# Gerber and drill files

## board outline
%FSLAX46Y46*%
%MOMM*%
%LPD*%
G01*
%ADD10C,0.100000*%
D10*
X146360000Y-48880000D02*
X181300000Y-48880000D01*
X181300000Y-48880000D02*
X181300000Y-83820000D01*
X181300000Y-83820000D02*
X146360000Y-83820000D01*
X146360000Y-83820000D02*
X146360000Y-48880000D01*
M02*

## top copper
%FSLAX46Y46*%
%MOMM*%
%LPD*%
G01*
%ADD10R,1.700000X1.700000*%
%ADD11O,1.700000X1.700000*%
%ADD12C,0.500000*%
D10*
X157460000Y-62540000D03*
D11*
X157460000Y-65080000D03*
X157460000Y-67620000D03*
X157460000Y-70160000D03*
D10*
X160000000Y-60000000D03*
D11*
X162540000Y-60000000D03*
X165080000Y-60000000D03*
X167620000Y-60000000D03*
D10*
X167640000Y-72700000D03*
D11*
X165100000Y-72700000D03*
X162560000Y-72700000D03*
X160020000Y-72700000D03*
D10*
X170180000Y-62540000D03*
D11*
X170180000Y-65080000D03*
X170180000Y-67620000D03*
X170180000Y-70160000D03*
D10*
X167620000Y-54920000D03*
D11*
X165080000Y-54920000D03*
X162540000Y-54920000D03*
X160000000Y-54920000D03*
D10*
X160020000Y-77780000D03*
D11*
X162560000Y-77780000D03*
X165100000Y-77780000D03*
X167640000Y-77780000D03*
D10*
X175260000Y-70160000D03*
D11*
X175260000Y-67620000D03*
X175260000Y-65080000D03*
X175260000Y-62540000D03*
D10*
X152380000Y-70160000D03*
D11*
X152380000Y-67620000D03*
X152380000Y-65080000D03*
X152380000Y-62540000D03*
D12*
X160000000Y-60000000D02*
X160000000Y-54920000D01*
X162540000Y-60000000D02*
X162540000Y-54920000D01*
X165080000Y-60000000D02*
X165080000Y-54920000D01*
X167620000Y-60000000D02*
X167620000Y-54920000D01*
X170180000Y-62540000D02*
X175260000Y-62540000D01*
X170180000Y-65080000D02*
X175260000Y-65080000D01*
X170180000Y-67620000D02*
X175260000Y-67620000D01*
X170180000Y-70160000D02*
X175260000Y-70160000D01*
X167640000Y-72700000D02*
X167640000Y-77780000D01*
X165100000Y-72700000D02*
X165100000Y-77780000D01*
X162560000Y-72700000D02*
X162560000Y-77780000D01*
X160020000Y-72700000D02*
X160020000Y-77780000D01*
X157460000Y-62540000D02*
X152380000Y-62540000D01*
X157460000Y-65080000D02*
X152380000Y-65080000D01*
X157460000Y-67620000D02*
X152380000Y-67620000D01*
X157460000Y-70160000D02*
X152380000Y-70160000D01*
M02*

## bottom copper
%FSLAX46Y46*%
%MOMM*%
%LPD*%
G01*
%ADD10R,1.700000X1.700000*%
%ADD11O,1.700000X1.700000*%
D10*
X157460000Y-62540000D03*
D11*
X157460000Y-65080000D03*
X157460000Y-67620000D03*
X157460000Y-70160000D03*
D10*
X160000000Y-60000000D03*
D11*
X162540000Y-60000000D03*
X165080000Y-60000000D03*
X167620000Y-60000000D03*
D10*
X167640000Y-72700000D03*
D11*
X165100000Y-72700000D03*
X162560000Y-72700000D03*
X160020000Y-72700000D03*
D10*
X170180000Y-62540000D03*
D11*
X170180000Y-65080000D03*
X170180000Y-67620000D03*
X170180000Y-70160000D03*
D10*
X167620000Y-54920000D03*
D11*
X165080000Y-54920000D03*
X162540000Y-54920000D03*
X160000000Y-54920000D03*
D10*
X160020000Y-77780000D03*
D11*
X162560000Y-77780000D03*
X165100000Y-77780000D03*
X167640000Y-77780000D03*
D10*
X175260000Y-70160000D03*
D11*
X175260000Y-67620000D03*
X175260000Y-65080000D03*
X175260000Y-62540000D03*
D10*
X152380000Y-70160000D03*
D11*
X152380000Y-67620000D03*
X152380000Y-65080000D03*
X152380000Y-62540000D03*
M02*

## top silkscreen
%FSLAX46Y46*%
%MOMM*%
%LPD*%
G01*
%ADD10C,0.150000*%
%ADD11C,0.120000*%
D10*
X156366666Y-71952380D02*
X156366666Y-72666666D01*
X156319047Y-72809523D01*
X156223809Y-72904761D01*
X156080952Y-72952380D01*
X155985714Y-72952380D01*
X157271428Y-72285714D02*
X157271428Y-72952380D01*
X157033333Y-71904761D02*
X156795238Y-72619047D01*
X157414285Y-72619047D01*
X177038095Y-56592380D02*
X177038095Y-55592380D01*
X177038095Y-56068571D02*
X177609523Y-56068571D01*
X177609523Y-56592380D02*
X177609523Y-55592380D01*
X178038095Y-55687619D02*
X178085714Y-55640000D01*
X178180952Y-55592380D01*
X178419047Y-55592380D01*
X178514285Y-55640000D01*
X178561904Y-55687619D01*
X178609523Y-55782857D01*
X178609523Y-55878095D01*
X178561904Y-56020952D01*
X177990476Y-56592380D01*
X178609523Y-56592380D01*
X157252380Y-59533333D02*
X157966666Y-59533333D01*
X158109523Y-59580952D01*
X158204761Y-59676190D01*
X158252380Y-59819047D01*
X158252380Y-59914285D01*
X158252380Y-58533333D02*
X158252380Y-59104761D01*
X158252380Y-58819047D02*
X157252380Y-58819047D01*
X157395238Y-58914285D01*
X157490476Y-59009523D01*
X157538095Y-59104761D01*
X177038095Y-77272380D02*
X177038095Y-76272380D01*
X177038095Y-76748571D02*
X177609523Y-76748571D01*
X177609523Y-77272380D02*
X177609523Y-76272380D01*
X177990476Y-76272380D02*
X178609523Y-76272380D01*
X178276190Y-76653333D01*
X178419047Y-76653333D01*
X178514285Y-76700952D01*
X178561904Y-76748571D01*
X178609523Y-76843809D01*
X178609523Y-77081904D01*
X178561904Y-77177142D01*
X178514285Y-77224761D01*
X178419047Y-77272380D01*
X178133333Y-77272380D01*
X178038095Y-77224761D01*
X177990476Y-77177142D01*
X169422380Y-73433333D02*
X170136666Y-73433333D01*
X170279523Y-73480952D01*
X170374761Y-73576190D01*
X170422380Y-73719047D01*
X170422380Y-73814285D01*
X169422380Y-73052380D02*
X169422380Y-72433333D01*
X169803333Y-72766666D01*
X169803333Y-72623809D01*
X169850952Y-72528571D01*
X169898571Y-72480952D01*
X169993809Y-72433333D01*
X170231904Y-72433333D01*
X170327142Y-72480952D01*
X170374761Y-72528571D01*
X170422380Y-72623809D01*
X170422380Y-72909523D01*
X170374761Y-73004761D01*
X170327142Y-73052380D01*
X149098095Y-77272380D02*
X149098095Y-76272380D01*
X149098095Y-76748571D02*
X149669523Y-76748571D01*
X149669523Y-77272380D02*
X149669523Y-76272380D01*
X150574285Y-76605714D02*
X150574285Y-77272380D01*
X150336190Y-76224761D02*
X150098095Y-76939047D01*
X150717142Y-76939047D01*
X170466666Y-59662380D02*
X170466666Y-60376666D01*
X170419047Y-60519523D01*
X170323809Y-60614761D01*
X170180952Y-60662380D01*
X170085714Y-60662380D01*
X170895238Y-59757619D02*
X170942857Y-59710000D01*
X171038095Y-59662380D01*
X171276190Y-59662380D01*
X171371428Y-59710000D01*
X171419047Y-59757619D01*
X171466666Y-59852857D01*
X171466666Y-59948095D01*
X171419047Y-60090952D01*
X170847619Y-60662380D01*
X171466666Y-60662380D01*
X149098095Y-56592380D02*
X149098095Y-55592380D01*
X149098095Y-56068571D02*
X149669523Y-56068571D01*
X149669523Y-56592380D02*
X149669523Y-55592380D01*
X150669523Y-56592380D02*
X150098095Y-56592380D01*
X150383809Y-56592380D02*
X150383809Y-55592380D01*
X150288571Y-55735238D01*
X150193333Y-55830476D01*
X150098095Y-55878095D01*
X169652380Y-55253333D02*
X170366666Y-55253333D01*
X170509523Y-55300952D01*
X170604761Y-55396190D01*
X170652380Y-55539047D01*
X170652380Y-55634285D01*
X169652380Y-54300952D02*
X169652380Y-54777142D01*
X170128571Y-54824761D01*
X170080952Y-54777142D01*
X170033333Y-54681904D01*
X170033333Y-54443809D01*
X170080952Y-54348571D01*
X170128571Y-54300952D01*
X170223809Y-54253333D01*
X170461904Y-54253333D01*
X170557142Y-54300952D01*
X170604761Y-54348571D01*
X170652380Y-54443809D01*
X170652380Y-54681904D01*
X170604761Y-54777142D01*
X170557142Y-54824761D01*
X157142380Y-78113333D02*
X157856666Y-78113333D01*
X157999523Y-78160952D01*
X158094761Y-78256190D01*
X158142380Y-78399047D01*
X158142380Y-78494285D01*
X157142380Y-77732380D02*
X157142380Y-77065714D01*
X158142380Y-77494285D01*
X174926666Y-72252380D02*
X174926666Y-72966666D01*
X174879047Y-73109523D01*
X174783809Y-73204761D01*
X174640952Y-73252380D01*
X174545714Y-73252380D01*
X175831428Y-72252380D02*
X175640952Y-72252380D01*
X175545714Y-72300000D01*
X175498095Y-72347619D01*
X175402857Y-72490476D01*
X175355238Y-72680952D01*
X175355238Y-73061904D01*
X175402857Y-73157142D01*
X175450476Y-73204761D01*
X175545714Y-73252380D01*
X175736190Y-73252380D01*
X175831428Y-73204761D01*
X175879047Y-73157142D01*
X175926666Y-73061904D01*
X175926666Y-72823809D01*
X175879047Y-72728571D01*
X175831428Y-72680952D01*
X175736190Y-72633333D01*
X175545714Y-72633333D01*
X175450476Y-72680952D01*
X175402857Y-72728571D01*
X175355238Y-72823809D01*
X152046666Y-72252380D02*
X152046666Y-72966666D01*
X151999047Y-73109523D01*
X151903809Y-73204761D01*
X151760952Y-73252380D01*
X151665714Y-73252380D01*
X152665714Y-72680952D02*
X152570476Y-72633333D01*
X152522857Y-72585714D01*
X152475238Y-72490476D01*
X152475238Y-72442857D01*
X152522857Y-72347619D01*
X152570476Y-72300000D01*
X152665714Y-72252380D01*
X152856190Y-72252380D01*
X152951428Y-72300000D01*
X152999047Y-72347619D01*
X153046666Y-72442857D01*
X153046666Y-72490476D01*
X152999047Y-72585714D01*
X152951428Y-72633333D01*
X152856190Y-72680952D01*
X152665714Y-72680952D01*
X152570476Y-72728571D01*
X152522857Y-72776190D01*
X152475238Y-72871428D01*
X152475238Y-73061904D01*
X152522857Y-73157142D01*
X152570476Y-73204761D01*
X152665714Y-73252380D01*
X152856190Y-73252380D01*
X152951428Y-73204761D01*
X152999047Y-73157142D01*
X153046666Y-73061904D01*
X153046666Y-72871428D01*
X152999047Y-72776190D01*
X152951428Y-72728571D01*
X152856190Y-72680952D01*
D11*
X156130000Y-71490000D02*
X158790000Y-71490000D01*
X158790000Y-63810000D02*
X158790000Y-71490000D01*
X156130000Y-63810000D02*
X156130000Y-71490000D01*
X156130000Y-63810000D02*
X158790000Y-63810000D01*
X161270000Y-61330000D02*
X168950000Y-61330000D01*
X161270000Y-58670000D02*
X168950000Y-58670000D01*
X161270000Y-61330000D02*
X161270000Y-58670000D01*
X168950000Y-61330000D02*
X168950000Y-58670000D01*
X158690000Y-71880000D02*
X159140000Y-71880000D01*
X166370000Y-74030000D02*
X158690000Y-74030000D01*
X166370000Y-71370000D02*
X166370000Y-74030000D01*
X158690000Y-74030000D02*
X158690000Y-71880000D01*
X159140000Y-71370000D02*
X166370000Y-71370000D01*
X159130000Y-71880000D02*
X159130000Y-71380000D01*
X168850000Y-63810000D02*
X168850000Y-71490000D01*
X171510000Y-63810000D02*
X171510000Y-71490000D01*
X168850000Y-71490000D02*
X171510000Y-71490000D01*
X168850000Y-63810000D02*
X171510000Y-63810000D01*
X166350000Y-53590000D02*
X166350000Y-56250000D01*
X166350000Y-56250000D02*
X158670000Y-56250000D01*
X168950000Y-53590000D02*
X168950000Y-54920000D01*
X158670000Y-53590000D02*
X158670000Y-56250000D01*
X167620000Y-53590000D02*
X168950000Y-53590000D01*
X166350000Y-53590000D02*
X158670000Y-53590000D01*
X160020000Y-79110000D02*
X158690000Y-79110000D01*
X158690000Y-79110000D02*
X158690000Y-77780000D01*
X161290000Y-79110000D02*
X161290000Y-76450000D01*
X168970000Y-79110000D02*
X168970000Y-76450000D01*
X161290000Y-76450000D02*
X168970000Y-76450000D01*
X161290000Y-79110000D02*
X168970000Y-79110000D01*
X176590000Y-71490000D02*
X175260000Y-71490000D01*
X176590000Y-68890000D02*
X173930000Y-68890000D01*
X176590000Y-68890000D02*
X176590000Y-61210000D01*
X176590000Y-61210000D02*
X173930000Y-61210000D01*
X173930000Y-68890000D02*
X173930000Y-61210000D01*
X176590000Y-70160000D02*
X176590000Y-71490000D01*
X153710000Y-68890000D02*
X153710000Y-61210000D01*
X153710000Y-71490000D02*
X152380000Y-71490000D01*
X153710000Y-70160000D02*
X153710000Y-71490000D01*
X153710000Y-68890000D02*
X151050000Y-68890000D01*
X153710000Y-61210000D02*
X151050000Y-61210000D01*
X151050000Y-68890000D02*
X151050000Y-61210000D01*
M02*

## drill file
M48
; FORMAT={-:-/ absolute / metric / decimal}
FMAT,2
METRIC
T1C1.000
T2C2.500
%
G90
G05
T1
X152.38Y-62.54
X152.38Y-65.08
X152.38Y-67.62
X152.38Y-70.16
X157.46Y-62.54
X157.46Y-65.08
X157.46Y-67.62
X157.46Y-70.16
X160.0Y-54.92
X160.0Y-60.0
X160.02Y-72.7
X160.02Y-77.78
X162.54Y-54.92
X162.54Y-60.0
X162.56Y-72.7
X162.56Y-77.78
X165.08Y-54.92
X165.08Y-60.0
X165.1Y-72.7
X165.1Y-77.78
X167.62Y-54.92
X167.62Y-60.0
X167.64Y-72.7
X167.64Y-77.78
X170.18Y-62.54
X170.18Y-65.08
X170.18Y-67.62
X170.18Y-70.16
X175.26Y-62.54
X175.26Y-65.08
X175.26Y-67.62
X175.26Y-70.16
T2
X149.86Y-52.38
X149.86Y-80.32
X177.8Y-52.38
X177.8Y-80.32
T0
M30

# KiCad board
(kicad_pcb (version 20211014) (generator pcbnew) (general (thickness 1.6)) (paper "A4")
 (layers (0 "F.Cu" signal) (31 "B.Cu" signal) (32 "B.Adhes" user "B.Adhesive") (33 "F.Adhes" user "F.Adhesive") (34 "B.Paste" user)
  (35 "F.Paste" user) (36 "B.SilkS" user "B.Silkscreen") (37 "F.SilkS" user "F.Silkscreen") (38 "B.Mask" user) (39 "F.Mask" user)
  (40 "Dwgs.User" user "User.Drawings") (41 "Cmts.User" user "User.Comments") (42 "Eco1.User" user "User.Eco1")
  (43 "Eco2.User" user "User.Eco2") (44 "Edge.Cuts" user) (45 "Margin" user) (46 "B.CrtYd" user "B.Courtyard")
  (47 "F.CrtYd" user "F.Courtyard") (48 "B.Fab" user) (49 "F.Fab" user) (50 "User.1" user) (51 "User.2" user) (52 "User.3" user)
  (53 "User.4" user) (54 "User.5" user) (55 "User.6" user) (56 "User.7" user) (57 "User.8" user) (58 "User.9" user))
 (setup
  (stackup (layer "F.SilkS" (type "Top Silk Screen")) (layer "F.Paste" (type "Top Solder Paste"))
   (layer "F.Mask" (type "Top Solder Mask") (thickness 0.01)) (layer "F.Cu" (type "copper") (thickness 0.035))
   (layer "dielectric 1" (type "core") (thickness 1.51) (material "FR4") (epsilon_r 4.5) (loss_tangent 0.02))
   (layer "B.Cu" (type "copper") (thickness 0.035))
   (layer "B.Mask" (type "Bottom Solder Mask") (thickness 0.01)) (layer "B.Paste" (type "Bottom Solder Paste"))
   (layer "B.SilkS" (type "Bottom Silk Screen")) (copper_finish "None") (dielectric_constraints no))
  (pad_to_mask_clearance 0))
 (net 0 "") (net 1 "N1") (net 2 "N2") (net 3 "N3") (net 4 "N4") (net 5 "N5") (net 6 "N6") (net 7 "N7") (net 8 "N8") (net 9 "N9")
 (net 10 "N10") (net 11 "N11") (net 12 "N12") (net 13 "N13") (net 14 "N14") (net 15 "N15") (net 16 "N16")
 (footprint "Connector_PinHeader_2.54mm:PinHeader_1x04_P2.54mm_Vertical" (layer "F.Cu") (at 157.46 62.54)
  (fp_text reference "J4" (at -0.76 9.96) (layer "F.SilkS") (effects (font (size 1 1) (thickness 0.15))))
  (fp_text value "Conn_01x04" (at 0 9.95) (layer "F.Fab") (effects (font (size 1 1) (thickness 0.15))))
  (fp_line (start -1.33 8.95) (end 1.33 8.95) (layer "F.SilkS") (width 0.12))
  (fp_line (start 1.33 1.27) (end 1.33 8.95) (layer "F.SilkS") (width 0.12))
  (fp_line (start -1.33 1.27) (end -1.33 8.95) (layer "F.SilkS") (width 0.12))
  (fp_line (start -1.33 1.27) (end 1.33 1.27) (layer "F.SilkS") (width 0.12))
  (pad "1" thru_hole rect (at 0 0) (size 1.7 1.7) (drill 1) (layers *.Cu *.Mask) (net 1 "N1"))
  (pad "2" thru_hole oval (at 0 2.54) (size 1.7 1.7) (drill 1) (layers *.Cu *.Mask) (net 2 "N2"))
  (pad "3" thru_hole oval (at 0 5.08) (size 1.7 1.7) (drill 1) (layers *.Cu *.Mask) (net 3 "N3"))
  (pad "4" thru_hole oval (at 0 7.62) (size 1.7 1.7) (drill 1) (layers *.Cu *.Mask) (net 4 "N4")))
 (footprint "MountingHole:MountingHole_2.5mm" (layer "F.Cu") (at 177.8 52.38)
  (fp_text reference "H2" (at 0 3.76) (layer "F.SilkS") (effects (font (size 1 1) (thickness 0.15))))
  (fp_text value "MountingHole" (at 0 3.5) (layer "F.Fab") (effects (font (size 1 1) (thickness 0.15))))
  (pad "" np_thru_hole circle (at 0 0) (size 2.5 2.5) (drill 2.5) (layers *.Cu *.Mask)))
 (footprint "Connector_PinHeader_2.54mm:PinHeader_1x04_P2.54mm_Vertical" (layer "F.Cu") (at 167.62 54.92 -90)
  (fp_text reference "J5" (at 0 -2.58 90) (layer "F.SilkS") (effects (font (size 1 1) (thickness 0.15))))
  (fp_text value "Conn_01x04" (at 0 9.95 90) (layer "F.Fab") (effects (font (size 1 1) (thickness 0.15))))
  (fp_line (start -1.33 1.27) (end 1.33 1.27) (layer "F.SilkS") (width 0.12))
  (fp_line (start 1.33 1.27) (end 1.33 8.95) (layer "F.SilkS") (width 0.12))
  (fp_line (start -1.33 -1.33) (end 0 -1.33) (layer "F.SilkS") (width 0.12))
  (fp_line (start -1.33 8.95) (end 1.33 8.95) (layer "F.SilkS") (width 0.12))
  (fp_line (start -1.33 0) (end -1.33 -1.33) (layer "F.SilkS") (width 0.12))
  (fp_line (start -1.33 1.27) (end -1.33 8.95) (layer "F.SilkS") (width 0.12))
  (pad "1" thru_hole rect (at 0 0 270) (size 1.7 1.7) (drill 1) (layers *.Cu *.Mask) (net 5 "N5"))
  (pad "2" thru_hole oval (at 0 2.54 270) (size 1.7 1.7) (drill 1) (layers *.Cu *.Mask) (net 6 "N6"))
  (pad "3" thru_hole oval (at 0 5.08 270) (size 1.7 1.7) (drill 1) (layers *.Cu *.Mask) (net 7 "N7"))
  (pad "4" thru_hole oval (at 0 7.62 270) (size 1.7 1.7) (drill 1) (layers *.Cu *.Mask) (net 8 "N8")))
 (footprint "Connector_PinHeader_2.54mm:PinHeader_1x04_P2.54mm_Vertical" (layer "F.Cu") (at 160 60 90)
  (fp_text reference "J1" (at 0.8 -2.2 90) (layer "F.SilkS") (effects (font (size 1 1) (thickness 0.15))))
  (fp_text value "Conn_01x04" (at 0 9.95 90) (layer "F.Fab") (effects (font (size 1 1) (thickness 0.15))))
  (fp_line (start -1.33 1.27) (end -1.33 8.95) (layer "F.SilkS") (width 0.12))
  (fp_line (start 1.33 1.27) (end 1.33 8.95) (layer "F.SilkS") (width 0.12))
  (fp_line (start -1.33 1.27) (end 1.33 1.27) (layer "F.SilkS") (width 0.12))
  (fp_line (start -1.33 8.95) (end 1.33 8.95) (layer "F.SilkS") (width 0.12))
  (pad "1" thru_hole rect (at 0 0 90) (size 1.7 1.7) (drill 1) (layers *.Cu *.Mask) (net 8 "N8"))
  (pad "2" thru_hole oval (at 0 2.54 90) (size 1.7 1.7) (drill 1) (layers *.Cu *.Mask) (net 7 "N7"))
  (pad "3" thru_hole oval (at 0 5.08 90) (size 1.7 1.7) (drill 1) (layers *.Cu *.Mask) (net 6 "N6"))
  (pad "4" thru_hole oval (at 0 7.62 90) (size 1.7 1.7) (drill 1) (layers *.Cu *.Mask) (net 5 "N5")))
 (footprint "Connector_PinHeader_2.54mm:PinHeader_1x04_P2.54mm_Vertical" (layer "F.Cu") (at 160.02 77.78 90)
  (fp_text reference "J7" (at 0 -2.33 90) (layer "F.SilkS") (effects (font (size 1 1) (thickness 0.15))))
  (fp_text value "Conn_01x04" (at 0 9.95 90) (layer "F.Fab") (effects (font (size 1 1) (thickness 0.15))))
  (fp_line (start -1.33 0) (end -1.33 -1.33) (layer "F.SilkS") (width 0.12))
  (fp_line (start -1.33 -1.33) (end 0 -1.33) (layer "F.SilkS") (width 0.12))
  (fp_line (start -1.33 1.27) (end 1.33 1.27) (layer "F.SilkS") (width 0.12))
  (fp_line (start -1.33 8.95) (end 1.33 8.95) (layer "F.SilkS") (width 0.12))
  (fp_line (start 1.33 1.27) (end 1.33 8.95) (layer "F.SilkS") (width 0.12))
  (fp_line (start -1.33 1.27) (end -1.33 8.95) (layer "F.SilkS") (width 0.12))
  (pad "1" thru_hole rect (at 0 0 90) (size 1.7 1.7) (drill 1) (layers *.Cu *.Mask) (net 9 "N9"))
  (pad "2" thru_hole oval (at 0 2.54 90) (size 1.7 1.7) (drill 1) (layers *.Cu *.Mask) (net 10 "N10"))
  (pad "3" thru_hole oval (at 0 5.08 90) (size 1.7 1.7) (drill 1) (layers *.Cu *.Mask) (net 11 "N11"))
  (pad "4" thru_hole oval (at 0 7.62 90) (size 1.7 1.7) (drill 1) (layers *.Cu *.Mask) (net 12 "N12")))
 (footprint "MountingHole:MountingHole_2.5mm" (layer "F.Cu") (at 177.8 80.32)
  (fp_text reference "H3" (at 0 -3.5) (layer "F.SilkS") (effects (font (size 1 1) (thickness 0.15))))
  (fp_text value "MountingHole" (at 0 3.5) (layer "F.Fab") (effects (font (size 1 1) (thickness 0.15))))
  (pad "" np_thru_hole circle (at 0 0) (size 2.5 2.5) (drill 2.5) (layers *.Cu *.Mask)))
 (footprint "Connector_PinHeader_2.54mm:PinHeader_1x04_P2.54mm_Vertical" (layer "F.Cu") (at 175.26 70.16 180)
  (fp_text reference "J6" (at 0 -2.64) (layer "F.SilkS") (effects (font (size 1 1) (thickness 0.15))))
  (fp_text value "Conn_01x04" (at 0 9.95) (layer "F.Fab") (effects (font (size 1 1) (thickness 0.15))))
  (fp_line (start -1.33 -1.33) (end 0 -1.33) (layer "F.SilkS") (width 0.12))
  (fp_line (start -1.33 1.27) (end 1.33 1.27) (layer "F.SilkS") (width 0.12))
  (fp_line (start -1.33 1.27) (end -1.33 8.95) (layer "F.SilkS") (width 0.12))
  (fp_line (start -1.33 8.95) (end 1.33 8.95) (layer "F.SilkS") (width 0.12))
  (fp_line (start 1.33 1.27) (end 1.33 8.95) (layer "F.SilkS") (width 0.12))
  (fp_line (start -1.33 0) (end -1.33 -1.33) (layer "F.SilkS") (width 0.12))
  (pad "1" thru_hole rect (at 0 0 180) (size 1.7 1.7) (drill 1) (layers *.Cu *.Mask) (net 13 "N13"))
  (pad "2" thru_hole oval (at 0 2.54 180) (size 1.7 1.7) (drill 1) (layers *.Cu *.Mask) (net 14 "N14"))
  (pad "3" thru_hole oval (at 0 5.08 180) (size 1.7 1.7) (drill 1) (layers *.Cu *.Mask) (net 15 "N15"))
  (pad "4" thru_hole oval (at 0 7.62 180) (size 1.7 1.7) (drill 1) (layers *.Cu *.Mask) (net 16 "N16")))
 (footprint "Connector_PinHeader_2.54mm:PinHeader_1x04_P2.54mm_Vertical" (layer "F.Cu") (at 167.64 72.7 -90)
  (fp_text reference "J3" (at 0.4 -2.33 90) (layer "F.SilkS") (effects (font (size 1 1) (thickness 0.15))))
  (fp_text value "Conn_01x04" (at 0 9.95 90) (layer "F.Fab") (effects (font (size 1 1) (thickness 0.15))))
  (fp_line (start -0.82 8.95) (end -0.82 8.5) (layer "F.SilkS") (width 0.12))
  (fp_line (start 1.33 1.27) (end 1.33 8.95) (layer "F.SilkS") (width 0.12))
  (fp_line (start -1.33 1.27) (end 1.33 1.27) (layer "F.SilkS") (width 0.12))
  (fp_line (start 1.33 8.95) (end -0.82 8.95) (layer "F.SilkS") (width 0.12))
  (fp_line (start -1.33 8.5) (end -1.33 1.27) (layer "F.SilkS") (width 0.12))
  (fp_line (start -0.82 8.51) (end -1.32 8.51) (layer "F.SilkS") (width 0.12))
  (pad "1" thru_hole rect (at 0 0 270) (size 1.7 1.7) (drill 1) (layers *.Cu *.Mask) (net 12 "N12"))
  (pad "2" thru_hole oval (at 0 2.54 270) (size 1.7 1.7) (drill 1) (layers *.Cu *.Mask) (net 11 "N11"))
  (pad "3" thru_hole oval (at 0 5.08 270) (size 1.7 1.7) (drill 1) (layers *.Cu *.Mask) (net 10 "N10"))
  (pad "4" thru_hole oval (at 0 7.62 270) (size 1.7 1.7) (drill 1) (layers *.Cu *.Mask) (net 9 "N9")))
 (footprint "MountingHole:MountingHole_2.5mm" (layer "F.Cu") (at 149.86 80.32)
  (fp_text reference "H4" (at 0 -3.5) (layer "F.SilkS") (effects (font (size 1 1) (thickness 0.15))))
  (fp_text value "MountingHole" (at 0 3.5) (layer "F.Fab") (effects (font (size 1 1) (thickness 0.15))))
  (pad "" np_thru_hole circle (at 0 0) (size 2.5 2.5) (drill 2.5) (layers *.Cu *.Mask)))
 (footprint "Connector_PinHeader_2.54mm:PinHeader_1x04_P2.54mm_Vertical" (layer "F.Cu") (at 170.18 62.54)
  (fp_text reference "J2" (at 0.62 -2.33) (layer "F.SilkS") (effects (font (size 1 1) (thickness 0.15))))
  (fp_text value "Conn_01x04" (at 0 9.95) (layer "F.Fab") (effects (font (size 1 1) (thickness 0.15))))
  (fp_line (start -1.33 1.27) (end -1.33 8.95) (layer "F.SilkS") (width 0.12))
  (fp_line (start 1.33 1.27) (end 1.33 8.95) (layer "F.SilkS") (width 0.12))
  (fp_line (start -1.33 8.95) (end 1.33 8.95) (layer "F.SilkS") (width 0.12))
  (fp_line (start -1.33 1.27) (end 1.33 1.27) (layer "F.SilkS") (width 0.12))
  (pad "1" thru_hole rect (at 0 0) (size 1.7 1.7) (drill 1) (layers *.Cu *.Mask) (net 16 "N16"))
  (pad "2" thru_hole oval (at 0 2.54) (size 1.7 1.7) (drill 1) (layers *.Cu *.Mask) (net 15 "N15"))
  (pad "3" thru_hole oval (at 0 5.08) (size 1.7 1.7) (drill 1) (layers *.Cu *.Mask) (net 14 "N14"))
  (pad "4" thru_hole oval (at 0 7.62) (size 1.7 1.7) (drill 1) (layers *.Cu *.Mask) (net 13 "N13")))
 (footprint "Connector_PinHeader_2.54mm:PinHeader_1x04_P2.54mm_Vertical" (layer "F.Cu") (at 152.38 70.16 180)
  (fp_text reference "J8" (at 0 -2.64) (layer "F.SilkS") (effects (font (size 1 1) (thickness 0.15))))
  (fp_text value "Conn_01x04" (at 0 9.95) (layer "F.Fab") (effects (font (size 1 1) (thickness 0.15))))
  (fp_line (start -1.33 1.27) (end -1.33 8.95) (layer "F.SilkS") (width 0.12))
  (fp_line (start -1.33 -1.33) (end 0 -1.33) (layer "F.SilkS") (width 0.12))
  (fp_line (start -1.33 0) (end -1.33 -1.33) (layer "F.SilkS") (width 0.12))
  (fp_line (start -1.33 1.27) (end 1.33 1.27) (layer "F.SilkS") (width 0.12))
  (fp_line (start -1.33 8.95) (end 1.33 8.95) (layer "F.SilkS") (width 0.12))
  (fp_line (start 1.33 1.27) (end 1.33 8.95) (layer "F.SilkS") (width 0.12))
  (pad "1" thru_hole rect (at 0 0 180) (size 1.7 1.7) (drill 1) (layers *.Cu *.Mask) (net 4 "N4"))
  (pad "2" thru_hole oval (at 0 2.54 180) (size 1.7 1.7) (drill 1) (layers *.Cu *.Mask) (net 3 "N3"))
  (pad "3" thru_hole oval (at 0 5.08 180) (size 1.7 1.7) (drill 1) (layers *.Cu *.Mask) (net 2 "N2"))
  (pad "4" thru_hole oval (at 0 7.62 180) (size 1.7 1.7) (drill 1) (layers *.Cu *.Mask) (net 1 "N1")))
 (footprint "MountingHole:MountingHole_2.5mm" (layer "F.Cu") (at 149.86 52.38)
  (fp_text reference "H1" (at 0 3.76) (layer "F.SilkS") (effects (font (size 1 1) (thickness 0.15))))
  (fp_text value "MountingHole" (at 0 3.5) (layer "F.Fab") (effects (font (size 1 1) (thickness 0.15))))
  (pad "" np_thru_hole circle (at 0 0) (size 2.5 2.5) (drill 2.5) (layers *.Cu *.Mask)))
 (gr_rect (start 146.36 48.88) (end 181.3 83.82) (layer "Edge.Cuts") (width 0.1) (fill none))
 (segment (start 160 60) (end 160 54.92) (width 0.5) (layer "F.Cu") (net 8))
 (segment (start 162.54 60) (end 162.54 54.92) (width 0.5) (layer "F.Cu") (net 7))
 (segment (start 165.08 60) (end 165.08 54.92) (width 0.5) (layer "F.Cu") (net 6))
 (segment (start 167.62 60) (end 167.62 54.92) (width 0.5) (layer "F.Cu") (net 5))
 (segment (start 170.18 62.54) (end 175.26 62.54) (width 0.5) (layer "F.Cu") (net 16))
 (segment (start 170.18 65.08) (end 175.26 65.08) (width 0.5) (layer "F.Cu") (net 15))
 (segment (start 170.18 67.62) (end 175.26 67.62) (width 0.5) (layer "F.Cu") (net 14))
 (segment (start 170.18 70.16) (end 175.26 70.16) (width 0.5) (layer "F.Cu") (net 13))
 (segment (start 167.64 72.7) (end 167.64 77.78) (width 0.5) (layer "F.Cu") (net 12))
 (segment (start 165.1 72.7) (end 165.1 77.78) (width 0.5) (layer "F.Cu") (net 11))
 (segment (start 162.56 72.7) (end 162.56 77.78) (width 0.5) (layer "F.Cu") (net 10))
 (segment (start 160.02 72.7) (end 160.02 77.78) (width 0.5) (layer "F.Cu") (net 9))
 (segment (start 157.46 62.54) (end 152.38 62.54) (width 0.5) (layer "F.Cu") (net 1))
 (segment (start 157.46 65.08) (end 152.38 65.08) (width 0.5) (layer "F.Cu") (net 2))
 (segment (start 157.46 67.62) (end 152.38 67.62) (width 0.5) (layer "F.Cu") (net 3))
 (segment (start 157.46 70.16) (end 152.38 70.16) (width 0.5) (layer "F.Cu") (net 4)))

